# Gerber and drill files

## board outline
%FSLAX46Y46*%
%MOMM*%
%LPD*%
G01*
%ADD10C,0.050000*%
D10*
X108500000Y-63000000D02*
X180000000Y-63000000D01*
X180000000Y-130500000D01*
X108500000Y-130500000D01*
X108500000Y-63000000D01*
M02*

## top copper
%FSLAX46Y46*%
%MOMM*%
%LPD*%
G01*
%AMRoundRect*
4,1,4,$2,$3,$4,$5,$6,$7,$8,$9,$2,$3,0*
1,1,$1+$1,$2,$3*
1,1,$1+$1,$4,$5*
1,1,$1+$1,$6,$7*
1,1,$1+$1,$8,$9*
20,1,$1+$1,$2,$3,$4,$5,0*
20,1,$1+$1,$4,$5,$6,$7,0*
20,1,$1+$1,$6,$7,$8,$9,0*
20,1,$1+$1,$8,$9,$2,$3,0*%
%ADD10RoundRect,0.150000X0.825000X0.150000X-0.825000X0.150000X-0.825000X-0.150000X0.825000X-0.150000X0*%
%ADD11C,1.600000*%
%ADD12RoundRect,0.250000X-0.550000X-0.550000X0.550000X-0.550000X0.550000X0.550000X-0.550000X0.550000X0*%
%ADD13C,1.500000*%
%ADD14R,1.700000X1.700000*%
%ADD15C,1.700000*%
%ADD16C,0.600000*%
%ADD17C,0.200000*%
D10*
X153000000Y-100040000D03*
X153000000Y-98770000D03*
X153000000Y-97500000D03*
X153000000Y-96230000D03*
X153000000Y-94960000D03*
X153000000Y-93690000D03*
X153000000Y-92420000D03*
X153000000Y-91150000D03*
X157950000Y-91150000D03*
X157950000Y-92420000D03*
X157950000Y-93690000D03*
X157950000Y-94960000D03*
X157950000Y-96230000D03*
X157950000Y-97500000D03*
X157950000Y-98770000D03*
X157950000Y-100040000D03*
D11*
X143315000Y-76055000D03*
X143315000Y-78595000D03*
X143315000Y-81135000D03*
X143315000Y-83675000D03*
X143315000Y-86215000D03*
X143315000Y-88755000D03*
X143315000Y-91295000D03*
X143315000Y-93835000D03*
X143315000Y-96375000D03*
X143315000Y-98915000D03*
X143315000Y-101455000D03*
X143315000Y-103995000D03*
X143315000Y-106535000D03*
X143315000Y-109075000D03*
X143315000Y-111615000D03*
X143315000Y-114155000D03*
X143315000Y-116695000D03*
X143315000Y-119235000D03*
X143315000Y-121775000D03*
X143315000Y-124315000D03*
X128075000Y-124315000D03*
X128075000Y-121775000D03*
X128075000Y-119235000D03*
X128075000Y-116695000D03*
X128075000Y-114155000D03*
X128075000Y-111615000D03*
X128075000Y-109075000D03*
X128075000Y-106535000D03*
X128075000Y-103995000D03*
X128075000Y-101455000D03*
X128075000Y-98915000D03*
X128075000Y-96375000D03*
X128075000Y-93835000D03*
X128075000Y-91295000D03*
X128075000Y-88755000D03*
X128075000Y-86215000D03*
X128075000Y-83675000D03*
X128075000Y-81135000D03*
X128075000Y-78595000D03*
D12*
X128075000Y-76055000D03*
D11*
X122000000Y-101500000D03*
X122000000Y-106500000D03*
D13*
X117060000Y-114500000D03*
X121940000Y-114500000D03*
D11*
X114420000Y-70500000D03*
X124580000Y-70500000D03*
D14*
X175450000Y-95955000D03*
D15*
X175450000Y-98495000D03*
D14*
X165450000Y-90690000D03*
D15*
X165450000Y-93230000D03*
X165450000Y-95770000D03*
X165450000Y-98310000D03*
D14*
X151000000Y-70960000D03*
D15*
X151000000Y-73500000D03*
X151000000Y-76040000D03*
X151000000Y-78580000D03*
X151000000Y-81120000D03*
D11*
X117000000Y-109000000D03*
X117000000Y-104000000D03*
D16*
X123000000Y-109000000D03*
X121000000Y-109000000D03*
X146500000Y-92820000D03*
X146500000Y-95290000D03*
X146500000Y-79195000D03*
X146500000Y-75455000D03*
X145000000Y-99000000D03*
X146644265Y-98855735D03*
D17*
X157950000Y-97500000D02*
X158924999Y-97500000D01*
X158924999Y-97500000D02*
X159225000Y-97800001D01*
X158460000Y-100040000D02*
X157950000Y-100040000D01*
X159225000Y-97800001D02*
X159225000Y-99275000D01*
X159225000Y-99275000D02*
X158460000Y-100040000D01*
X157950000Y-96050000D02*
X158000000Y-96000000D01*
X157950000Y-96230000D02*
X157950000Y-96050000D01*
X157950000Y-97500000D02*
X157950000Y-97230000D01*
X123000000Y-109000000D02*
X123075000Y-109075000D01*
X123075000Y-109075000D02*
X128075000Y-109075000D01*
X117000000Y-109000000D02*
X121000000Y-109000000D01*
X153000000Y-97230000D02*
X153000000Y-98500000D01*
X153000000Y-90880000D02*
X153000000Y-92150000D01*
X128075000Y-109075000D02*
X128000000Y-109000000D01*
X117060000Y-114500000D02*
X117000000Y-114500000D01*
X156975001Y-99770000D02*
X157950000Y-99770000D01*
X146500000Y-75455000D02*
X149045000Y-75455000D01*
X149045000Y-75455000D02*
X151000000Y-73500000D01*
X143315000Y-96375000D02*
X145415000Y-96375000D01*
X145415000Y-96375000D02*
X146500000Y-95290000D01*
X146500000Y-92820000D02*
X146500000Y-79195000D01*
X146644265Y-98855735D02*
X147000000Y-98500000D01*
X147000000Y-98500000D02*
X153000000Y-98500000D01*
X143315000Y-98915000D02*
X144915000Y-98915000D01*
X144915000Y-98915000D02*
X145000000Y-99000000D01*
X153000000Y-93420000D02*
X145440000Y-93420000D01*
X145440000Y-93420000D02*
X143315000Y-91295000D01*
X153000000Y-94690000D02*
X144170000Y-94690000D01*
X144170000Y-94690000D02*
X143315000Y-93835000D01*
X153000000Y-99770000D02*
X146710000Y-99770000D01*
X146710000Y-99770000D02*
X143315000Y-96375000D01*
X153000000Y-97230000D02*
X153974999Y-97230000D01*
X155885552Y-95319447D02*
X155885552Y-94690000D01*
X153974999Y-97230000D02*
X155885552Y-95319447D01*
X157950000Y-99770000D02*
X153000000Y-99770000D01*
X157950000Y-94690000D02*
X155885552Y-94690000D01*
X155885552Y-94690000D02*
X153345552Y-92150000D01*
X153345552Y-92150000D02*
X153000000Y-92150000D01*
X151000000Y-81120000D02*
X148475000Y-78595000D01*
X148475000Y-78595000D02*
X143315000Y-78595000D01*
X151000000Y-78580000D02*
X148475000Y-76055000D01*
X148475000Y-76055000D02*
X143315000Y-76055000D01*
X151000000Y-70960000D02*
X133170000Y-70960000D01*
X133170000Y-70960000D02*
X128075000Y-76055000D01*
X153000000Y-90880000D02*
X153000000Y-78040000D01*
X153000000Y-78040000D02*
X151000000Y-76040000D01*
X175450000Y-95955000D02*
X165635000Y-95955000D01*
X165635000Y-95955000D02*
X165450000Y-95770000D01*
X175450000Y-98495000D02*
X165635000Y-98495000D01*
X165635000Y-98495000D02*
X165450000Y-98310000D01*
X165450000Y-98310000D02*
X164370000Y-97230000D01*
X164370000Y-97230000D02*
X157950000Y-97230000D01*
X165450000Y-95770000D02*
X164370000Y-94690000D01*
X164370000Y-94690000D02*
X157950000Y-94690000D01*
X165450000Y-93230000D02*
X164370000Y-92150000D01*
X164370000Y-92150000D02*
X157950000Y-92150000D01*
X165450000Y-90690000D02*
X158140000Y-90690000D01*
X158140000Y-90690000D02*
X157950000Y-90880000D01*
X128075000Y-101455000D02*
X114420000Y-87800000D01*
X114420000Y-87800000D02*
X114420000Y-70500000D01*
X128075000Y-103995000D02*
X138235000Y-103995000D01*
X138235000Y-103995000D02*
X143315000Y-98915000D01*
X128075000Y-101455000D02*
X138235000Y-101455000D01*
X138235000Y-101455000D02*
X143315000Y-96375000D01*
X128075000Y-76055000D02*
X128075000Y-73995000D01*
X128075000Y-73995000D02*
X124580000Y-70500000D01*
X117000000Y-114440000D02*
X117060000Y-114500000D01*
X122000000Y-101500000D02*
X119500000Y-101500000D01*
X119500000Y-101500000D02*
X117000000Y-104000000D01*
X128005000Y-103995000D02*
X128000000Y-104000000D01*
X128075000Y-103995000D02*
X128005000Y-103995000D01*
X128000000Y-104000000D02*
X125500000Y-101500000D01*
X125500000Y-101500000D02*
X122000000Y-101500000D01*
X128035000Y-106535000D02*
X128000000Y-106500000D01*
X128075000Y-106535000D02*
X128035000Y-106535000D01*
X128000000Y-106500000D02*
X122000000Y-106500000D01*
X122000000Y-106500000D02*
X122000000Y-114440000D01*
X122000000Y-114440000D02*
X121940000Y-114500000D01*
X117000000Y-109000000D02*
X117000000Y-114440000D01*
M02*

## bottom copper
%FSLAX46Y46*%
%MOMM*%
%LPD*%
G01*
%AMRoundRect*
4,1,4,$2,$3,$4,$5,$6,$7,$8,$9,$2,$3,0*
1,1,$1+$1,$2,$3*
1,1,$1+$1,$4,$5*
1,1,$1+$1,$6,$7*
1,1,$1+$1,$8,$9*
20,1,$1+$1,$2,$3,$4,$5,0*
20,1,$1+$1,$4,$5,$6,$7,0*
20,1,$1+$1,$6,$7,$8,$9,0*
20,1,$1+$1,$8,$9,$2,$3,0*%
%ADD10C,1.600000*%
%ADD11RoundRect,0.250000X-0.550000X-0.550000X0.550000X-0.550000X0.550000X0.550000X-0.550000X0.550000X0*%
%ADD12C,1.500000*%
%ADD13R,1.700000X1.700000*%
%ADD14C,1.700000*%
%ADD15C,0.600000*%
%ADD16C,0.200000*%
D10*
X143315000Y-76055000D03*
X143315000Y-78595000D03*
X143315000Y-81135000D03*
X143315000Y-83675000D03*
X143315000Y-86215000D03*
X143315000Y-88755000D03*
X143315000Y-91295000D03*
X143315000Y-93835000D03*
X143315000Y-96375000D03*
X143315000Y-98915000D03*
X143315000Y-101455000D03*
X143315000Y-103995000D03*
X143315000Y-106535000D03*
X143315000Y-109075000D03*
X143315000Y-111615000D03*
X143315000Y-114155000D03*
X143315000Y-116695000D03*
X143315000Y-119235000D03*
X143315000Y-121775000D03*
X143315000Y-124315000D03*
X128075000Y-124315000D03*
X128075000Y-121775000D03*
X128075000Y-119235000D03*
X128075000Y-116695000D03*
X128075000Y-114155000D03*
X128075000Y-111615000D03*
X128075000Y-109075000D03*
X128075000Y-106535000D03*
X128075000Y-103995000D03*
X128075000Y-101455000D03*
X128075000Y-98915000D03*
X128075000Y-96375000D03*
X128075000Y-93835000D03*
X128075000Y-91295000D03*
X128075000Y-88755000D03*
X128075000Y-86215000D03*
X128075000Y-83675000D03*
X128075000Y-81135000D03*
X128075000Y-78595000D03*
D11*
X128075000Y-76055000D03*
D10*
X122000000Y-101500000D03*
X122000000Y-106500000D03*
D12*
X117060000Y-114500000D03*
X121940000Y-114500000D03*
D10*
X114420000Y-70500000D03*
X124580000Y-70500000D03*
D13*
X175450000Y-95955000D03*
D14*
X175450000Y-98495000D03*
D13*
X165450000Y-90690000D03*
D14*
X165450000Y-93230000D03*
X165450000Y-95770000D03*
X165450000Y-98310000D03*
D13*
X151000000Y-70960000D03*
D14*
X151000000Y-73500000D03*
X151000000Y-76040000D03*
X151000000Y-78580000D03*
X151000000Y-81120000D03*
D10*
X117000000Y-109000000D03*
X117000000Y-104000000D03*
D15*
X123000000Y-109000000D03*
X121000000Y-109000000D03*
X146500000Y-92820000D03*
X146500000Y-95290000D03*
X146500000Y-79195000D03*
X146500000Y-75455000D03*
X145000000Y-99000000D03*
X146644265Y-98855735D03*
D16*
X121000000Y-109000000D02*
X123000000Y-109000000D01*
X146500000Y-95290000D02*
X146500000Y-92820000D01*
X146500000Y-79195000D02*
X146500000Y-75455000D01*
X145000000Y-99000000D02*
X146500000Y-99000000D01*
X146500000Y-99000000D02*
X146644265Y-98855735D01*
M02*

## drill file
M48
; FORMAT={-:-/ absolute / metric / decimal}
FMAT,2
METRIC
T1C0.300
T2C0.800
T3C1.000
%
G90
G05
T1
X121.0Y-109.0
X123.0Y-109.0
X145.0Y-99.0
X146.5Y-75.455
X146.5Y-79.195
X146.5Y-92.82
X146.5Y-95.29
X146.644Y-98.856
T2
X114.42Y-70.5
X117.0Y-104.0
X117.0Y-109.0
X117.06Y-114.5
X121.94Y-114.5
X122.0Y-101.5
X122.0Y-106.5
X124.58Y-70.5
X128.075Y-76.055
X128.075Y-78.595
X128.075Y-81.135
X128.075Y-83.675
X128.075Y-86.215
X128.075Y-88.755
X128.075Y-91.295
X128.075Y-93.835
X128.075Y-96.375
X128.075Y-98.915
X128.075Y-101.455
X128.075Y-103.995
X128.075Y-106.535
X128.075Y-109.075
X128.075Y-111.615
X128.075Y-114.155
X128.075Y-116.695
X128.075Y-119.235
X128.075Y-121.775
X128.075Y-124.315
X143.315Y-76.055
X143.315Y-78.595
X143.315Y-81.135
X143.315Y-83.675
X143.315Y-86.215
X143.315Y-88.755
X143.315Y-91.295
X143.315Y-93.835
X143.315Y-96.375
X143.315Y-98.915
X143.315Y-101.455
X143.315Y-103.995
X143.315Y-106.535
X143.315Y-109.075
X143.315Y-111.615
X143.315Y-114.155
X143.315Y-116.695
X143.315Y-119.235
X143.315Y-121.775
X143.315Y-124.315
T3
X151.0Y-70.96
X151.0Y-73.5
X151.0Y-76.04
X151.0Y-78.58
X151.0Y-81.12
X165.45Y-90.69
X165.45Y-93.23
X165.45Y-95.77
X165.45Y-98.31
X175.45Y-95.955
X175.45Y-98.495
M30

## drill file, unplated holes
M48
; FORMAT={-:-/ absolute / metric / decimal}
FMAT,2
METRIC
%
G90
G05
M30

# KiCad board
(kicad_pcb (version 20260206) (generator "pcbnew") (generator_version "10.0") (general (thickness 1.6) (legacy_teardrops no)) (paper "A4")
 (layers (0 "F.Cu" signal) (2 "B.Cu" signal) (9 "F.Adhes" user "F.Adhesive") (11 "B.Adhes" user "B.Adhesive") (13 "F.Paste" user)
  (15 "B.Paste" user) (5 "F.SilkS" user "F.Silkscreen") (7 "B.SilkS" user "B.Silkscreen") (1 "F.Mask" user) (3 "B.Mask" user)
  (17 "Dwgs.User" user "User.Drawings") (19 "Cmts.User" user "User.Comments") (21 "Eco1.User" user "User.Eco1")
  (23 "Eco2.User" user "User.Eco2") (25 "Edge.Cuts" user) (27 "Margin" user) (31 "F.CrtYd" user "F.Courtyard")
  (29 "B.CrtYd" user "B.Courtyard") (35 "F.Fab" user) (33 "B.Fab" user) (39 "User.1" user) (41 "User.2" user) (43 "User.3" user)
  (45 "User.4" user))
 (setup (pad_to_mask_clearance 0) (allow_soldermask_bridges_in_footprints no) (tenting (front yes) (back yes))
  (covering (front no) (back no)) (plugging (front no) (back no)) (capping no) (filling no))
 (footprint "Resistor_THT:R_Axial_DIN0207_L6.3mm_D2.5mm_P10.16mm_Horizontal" (layer "F.Cu") (at 114.42 70.5)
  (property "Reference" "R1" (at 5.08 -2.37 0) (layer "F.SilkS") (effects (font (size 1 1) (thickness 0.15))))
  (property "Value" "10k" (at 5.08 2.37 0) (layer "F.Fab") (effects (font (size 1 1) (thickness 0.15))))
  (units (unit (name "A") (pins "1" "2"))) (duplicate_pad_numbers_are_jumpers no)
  (pad "1" thru_hole circle (at 0 0) (size 1.6 1.6) (drill 0.8) (layers "*.Cu" "*.Mask") (remove_unused_layers no) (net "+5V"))
  (pad "2" thru_hole circle (at 10.16 0) (size 1.6 1.6) (drill 0.8) (layers "*.Cu" "*.Mask") (remove_unused_layers no)
   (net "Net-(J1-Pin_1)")))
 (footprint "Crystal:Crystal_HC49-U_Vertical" (layer "F.Cu") (at 117.06 114.5)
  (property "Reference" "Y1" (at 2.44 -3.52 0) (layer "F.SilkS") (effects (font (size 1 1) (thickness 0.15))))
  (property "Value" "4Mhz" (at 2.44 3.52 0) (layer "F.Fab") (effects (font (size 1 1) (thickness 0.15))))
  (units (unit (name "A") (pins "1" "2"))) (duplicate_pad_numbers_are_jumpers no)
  (pad "1" thru_hole circle (at 0 0) (size 1.5 1.5) (drill 0.8) (layers "*.Cu" "*.Mask") (remove_unused_layers no)
   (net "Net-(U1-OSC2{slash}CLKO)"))
  (pad "2" thru_hole circle (at 4.88 0) (size 1.5 1.5) (drill 0.8) (layers "*.Cu" "*.Mask") (remove_unused_layers no)
   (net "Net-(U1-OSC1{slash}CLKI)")))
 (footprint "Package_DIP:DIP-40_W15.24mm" (layer "F.Cu") (at 128.075 76.055)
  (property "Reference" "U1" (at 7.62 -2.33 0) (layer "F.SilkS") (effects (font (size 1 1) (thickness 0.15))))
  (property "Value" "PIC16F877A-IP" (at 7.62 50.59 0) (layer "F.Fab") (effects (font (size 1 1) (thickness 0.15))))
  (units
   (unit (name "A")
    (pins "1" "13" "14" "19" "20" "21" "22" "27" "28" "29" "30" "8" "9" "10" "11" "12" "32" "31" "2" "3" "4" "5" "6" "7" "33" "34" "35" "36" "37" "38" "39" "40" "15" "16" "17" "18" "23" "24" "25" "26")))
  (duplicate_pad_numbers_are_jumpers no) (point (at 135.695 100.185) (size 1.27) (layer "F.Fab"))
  (pad "1" thru_hole roundrect (at 0 0) (size 1.6 1.6) (drill 0.8) (layers "*.Cu" "*.Mask") (remove_unused_layers no)
   (roundrect_rratio 0.15625) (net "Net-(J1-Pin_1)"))
  (pad "2" thru_hole circle (at 0 2.54) (size 1.6 1.6) (drill 0.8) (layers "*.Cu" "*.Mask") (remove_unused_layers no)
   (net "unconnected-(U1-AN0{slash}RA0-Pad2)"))
  (pad "3" thru_hole circle (at 0 5.08) (size 1.6 1.6) (drill 0.8) (layers "*.Cu" "*.Mask") (remove_unused_layers no)
   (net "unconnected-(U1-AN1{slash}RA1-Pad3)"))
  (pad "4" thru_hole circle (at 0 7.62) (size 1.6 1.6) (drill 0.8) (layers "*.Cu" "*.Mask") (remove_unused_layers no)
   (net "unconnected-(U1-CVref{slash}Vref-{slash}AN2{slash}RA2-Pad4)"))
  (pad "5" thru_hole circle (at 0 10.16) (size 1.6 1.6) (drill 0.8) (layers "*.Cu" "*.Mask") (remove_unused_layers no)
   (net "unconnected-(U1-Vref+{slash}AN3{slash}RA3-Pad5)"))
  (pad "6" thru_hole circle (at 0 12.7) (size 1.6 1.6) (drill 0.8) (layers "*.Cu" "*.Mask") (remove_unused_layers no)
   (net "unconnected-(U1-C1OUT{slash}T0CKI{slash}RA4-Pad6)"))
  (pad "7" thru_hole circle (at 0 15.24) (size 1.6 1.6) (drill 0.8) (layers "*.Cu" "*.Mask") (remove_unused_layers no)
   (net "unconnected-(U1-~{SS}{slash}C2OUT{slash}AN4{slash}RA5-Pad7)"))
  (pad "8" thru_hole circle (at 0 17.78) (size 1.6 1.6) (drill 0.8) (layers "*.Cu" "*.Mask") (remove_unused_layers no)
   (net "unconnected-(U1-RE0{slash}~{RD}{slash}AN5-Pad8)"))
  (pad "9" thru_hole circle (at 0 20.32) (size 1.6 1.6) (drill 0.8) (layers "*.Cu" "*.Mask") (remove_unused_layers no)
   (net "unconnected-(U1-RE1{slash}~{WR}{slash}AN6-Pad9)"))
  (pad "10" thru_hole circle (at 0 22.86) (size 1.6 1.6) (drill 0.8) (layers "*.Cu" "*.Mask") (remove_unused_layers no)
   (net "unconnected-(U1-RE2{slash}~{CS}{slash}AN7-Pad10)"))
  (pad "11" thru_hole circle (at 0 25.4) (size 1.6 1.6) (drill 0.8) (layers "*.Cu" "*.Mask") (remove_unused_layers no) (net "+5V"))
  (pad "12" thru_hole circle (at 0 27.94) (size 1.6 1.6) (drill 0.8) (layers "*.Cu" "*.Mask") (remove_unused_layers no) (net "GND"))
  (pad "13" thru_hole circle (at 0 30.48) (size 1.6 1.6) (drill 0.8) (layers "*.Cu" "*.Mask") (remove_unused_layers no)
   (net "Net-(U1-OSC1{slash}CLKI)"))
  (pad "14" thru_hole circle (at 0 33.02) (size 1.6 1.6) (drill 0.8) (layers "*.Cu" "*.Mask") (remove_unused_layers no)
   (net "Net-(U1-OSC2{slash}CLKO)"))
  (pad "15" thru_hole circle (at 0 35.56) (size 1.6 1.6) (drill 0.8) (layers "*.Cu" "*.Mask") (remove_unused_layers no)
   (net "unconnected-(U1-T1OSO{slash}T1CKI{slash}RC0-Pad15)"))
  (pad "16" thru_hole circle (at 0 38.1) (size 1.6 1.6) (drill 0.8) (layers "*.Cu" "*.Mask") (remove_unused_layers no)
   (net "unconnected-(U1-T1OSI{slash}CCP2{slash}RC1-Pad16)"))
  (pad "17" thru_hole circle (at 0 40.64) (size 1.6 1.6) (drill 0.8) (layers "*.Cu" "*.Mask") (remove_unused_layers no)
   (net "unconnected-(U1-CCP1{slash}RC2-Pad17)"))
  (pad "18" thru_hole circle (at 0 43.18) (size 1.6 1.6) (drill 0.8) (layers "*.Cu" "*.Mask") (remove_unused_layers no)
   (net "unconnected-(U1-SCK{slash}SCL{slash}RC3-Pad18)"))
  (pad "19" thru_hole circle (at 0 45.72) (size 1.6 1.6) (drill 0.8) (layers "*.Cu" "*.Mask") (remove_unused_layers no)
   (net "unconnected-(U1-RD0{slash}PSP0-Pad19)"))
  (pad "20" thru_hole circle (at 0 48.26) (size 1.6 1.6) (drill 0.8) (layers "*.Cu" "*.Mask") (remove_unused_layers no)
   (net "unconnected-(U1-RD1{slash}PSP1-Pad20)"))
  (pad "21" thru_hole circle (at 15.24 48.26) (size 1.6 1.6) (drill 0.8) (layers "*.Cu" "*.Mask") (remove_unused_layers no)
   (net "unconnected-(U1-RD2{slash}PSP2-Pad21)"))
  (pad "22" thru_hole circle (at 15.24 45.72) (size 1.6 1.6) (drill 0.8) (layers "*.Cu" "*.Mask") (remove_unused_layers no)
   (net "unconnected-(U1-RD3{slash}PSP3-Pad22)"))
  (pad "23" thru_hole circle (at 15.24 43.18) (size 1.6 1.6) (drill 0.8) (layers "*.Cu" "*.Mask") (remove_unused_layers no)
   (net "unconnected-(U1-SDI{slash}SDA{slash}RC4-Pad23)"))
  (pad "24" thru_hole circle (at 15.24 40.64) (size 1.6 1.6) (drill 0.8) (layers "*.Cu" "*.Mask") (remove_unused_layers no)
   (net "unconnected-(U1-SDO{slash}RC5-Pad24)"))
  (pad "25" thru_hole circle (at 15.24 38.1) (size 1.6 1.6) (drill 0.8) (layers "*.Cu" "*.Mask") (remove_unused_layers no)
   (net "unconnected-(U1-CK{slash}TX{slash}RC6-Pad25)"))
  (pad "26" thru_hole circle (at 15.24 35.56) (size 1.6 1.6) (drill 0.8) (layers "*.Cu" "*.Mask") (remove_unused_layers no)
   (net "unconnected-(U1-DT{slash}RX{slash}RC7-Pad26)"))
  (pad "27" thru_hole circle (at 15.24 33.02) (size 1.6 1.6) (drill 0.8) (layers "*.Cu" "*.Mask") (remove_unused_layers no)
   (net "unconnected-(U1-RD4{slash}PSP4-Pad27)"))
  (pad "28" thru_hole circle (at 15.24 30.48) (size 1.6 1.6) (drill 0.8) (layers "*.Cu" "*.Mask") (remove_unused_layers no)
   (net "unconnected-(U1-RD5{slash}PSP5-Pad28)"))
  (pad "29" thru_hole circle (at 15.24 27.94) (size 1.6 1.6) (drill 0.8) (layers "*.Cu" "*.Mask") (remove_unused_layers no)
   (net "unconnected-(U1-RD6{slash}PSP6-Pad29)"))
  (pad "30" thru_hole circle (at 15.24 25.4) (size 1.6 1.6) (drill 0.8) (layers "*.Cu" "*.Mask") (remove_unused_layers no)
   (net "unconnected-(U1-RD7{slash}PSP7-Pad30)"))
  (pad "31" thru_hole circle (at 15.24 22.86) (size 1.6 1.6) (drill 0.8) (layers "*.Cu" "*.Mask") (remove_unused_layers no) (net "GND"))
  (pad "32" thru_hole circle (at 15.24 20.32) (size 1.6 1.6) (drill 0.8) (layers "*.Cu" "*.Mask") (remove_unused_layers no) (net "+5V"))
  (pad "33" thru_hole circle (at 15.24 17.78) (size 1.6 1.6) (drill 0.8) (layers "*.Cu" "*.Mask") (remove_unused_layers no)
   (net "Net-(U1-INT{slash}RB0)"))
  (pad "34" thru_hole circle (at 15.24 15.24) (size 1.6 1.6) (drill 0.8) (layers "*.Cu" "*.Mask") (remove_unused_layers no)
   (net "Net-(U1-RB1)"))
  (pad "35" thru_hole circle (at 15.24 12.7) (size 1.6 1.6) (drill 0.8) (layers "*.Cu" "*.Mask") (remove_unused_layers no)
   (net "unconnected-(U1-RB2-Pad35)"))
  (pad "36" thru_hole circle (at 15.24 10.16) (size 1.6 1.6) (drill 0.8) (layers "*.Cu" "*.Mask") (remove_unused_layers no)
   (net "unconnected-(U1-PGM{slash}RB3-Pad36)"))
  (pad "37" thru_hole circle (at 15.24 7.62) (size 1.6 1.6) (drill 0.8) (layers "*.Cu" "*.Mask") (remove_unused_layers no)
   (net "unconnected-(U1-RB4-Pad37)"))
  (pad "38" thru_hole circle (at 15.24 5.08) (size 1.6 1.6) (drill 0.8) (layers "*.Cu" "*.Mask") (remove_unused_layers no)
   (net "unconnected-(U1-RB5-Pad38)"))
  (pad "39" thru_hole circle (at 15.24 2.54) (size 1.6 1.6) (drill 0.8) (layers "*.Cu" "*.Mask") (remove_unused_layers no)
   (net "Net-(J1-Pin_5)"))
  (pad "40" thru_hole circle (at 15.24 0) (size 1.6 1.6) (drill 0.8) (layers "*.Cu" "*.Mask") (remove_unused_layers no)
   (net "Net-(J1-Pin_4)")))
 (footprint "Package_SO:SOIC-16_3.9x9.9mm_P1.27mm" (layer "F.Cu") (at 155.475 95.595 180)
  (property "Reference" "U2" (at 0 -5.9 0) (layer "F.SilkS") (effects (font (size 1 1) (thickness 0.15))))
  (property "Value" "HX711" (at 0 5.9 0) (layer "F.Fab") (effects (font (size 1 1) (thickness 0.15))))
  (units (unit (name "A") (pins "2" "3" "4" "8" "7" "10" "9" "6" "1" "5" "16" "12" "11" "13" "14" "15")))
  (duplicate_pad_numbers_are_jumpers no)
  (pad "1" smd roundrect (at -2.475 -4.445 180) (size 1.95 0.6) (layers "F.Cu" "F.Mask" "F.Paste") (roundrect_rratio 0.25) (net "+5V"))
  (pad "2" smd roundrect (at -2.475 -3.175 180) (size 1.95 0.6) (layers "F.Cu" "F.Mask" "F.Paste") (roundrect_rratio 0.25)
   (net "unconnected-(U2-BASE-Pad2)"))
  (pad "3" smd roundrect (at -2.475 -1.905 180) (size 1.95 0.6) (layers "F.Cu" "F.Mask" "F.Paste") (roundrect_rratio 0.25) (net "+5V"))
  (pad "4" smd roundrect (at -2.475 -0.635 180) (size 1.95 0.6) (layers "F.Cu" "F.Mask" "F.Paste") (roundrect_rratio 0.25)
   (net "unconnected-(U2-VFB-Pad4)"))
  (pad "5" smd roundrect (at -2.475 0.635 180) (size 1.95 0.6) (layers "F.Cu" "F.Mask" "F.Paste") (roundrect_rratio 0.25) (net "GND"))
  (pad "6" smd roundrect (at -2.475 1.905 180) (size 1.95 0.6) (layers "F.Cu" "F.Mask" "F.Paste") (roundrect_rratio 0.25)
   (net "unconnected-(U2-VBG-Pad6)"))
  (pad "7" smd roundrect (at -2.475 3.175 180) (size 1.95 0.6) (layers "F.Cu" "F.Mask" "F.Paste") (roundrect_rratio 0.25)
   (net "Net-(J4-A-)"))
  (pad "8" smd roundrect (at -2.475 4.445 180) (size 1.95 0.6) (layers "F.Cu" "F.Mask" "F.Paste") (roundrect_rratio 0.25)
   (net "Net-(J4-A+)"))
  (pad "9" smd roundrect (at 2.475 4.445 180) (size 1.95 0.6) (layers "F.Cu" "F.Mask" "F.Paste") (roundrect_rratio 0.25) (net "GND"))
  (pad "10" smd roundrect (at 2.475 3.175 180) (size 1.95 0.6) (layers "F.Cu" "F.Mask" "F.Paste") (roundrect_rratio 0.25) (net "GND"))
  (pad "11" smd roundrect (at 2.475 1.905 180) (size 1.95 0.6) (layers "F.Cu" "F.Mask" "F.Paste") (roundrect_rratio 0.25)
   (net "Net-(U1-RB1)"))
  (pad "12" smd roundrect (at 2.475 0.635 180) (size 1.95 0.6) (layers "F.Cu" "F.Mask" "F.Paste") (roundrect_rratio 0.25)
   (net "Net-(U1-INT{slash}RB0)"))
  (pad "13" smd roundrect (at 2.475 -0.635 180) (size 1.95 0.6) (layers "F.Cu" "F.Mask" "F.Paste") (roundrect_rratio 0.25)
   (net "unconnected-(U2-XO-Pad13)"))
  (pad "14" smd roundrect (at 2.475 -1.905 180) (size 1.95 0.6) (layers "F.Cu" "F.Mask" "F.Paste") (roundrect_rratio 0.25) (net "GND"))
  (pad "15" smd roundrect (at 2.475 -3.175 180) (size 1.95 0.6) (layers "F.Cu" "F.Mask" "F.Paste") (roundrect_rratio 0.25) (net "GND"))
  (pad "16" smd roundrect (at 2.475 -4.445 180) (size 1.95 0.6) (layers "F.Cu" "F.Mask" "F.Paste") (roundrect_rratio 0.25) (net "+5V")))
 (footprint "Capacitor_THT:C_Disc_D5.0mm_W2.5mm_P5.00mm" (layer "F.Cu") (at 117 109 90)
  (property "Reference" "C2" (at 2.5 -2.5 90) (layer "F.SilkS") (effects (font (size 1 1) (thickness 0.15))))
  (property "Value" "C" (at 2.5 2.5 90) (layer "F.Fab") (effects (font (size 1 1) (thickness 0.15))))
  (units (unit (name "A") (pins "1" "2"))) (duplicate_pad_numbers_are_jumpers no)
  (pad "1" thru_hole circle (at 0 0 90) (size 1.6 1.6) (drill 0.8) (layers "*.Cu" "*.Mask") (remove_unused_layers no)
   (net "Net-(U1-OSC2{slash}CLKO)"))
  (pad "2" thru_hole circle (at 5 0 90) (size 1.6 1.6) (drill 0.8) (layers "*.Cu" "*.Mask") (remove_unused_layers no) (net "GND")))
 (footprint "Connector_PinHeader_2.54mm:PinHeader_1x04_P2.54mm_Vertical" (layer "F.Cu") (at 165.45 90.69)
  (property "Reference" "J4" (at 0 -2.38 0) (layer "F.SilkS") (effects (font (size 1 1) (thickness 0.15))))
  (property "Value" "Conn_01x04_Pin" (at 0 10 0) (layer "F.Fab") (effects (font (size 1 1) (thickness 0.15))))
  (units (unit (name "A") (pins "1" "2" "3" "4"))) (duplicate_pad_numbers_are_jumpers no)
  (pad "1" thru_hole rect (at 0 0) (size 1.7 1.7) (drill 1) (layers "*.Cu" "*.Mask") (remove_unused_layers no) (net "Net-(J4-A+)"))
  (pad "2" thru_hole circle (at 0 2.54) (size 1.7 1.7) (drill 1) (layers "*.Cu" "*.Mask") (remove_unused_layers no) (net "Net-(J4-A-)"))
  (pad "3" thru_hole circle (at 0 5.08) (size 1.7 1.7) (drill 1) (layers "*.Cu" "*.Mask") (remove_unused_layers no) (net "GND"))
  (pad "4" thru_hole circle (at 0 7.62) (size 1.7 1.7) (drill 1) (layers "*.Cu" "*.Mask") (remove_unused_layers no) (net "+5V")))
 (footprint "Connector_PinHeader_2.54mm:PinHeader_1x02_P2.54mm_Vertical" (layer "F.Cu") (at 175.45 95.955)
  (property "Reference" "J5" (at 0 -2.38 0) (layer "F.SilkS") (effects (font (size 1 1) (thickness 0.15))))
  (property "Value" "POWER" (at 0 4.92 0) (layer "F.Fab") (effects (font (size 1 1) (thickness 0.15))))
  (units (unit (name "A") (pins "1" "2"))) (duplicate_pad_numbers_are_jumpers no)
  (pad "1" thru_hole rect (at 0 0) (size 1.7 1.7) (drill 1) (layers "*.Cu" "*.Mask") (remove_unused_layers no) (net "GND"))
  (pad "2" thru_hole circle (at 0 2.54) (size 1.7 1.7) (drill 1) (layers "*.Cu" "*.Mask") (remove_unused_layers no) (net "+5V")))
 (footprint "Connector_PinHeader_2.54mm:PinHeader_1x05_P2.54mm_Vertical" (layer "F.Cu") (at 151 70.96)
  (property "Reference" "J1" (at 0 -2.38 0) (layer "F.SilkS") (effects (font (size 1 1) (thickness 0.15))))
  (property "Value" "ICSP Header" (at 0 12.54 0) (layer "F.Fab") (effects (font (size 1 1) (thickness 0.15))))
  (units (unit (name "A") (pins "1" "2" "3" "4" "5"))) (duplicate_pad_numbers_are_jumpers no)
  (pad "1" thru_hole rect (at 0 0) (size 1.7 1.7) (drill 1) (layers "*.Cu" "*.Mask") (remove_unused_layers no) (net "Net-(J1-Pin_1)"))
  (pad "2" thru_hole circle (at 0 2.54) (size 1.7 1.7) (drill 1) (layers "*.Cu" "*.Mask") (remove_unused_layers no) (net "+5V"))
  (pad "3" thru_hole circle (at 0 5.08) (size 1.7 1.7) (drill 1) (layers "*.Cu" "*.Mask") (remove_unused_layers no) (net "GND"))
  (pad "4" thru_hole circle (at 0 7.62) (size 1.7 1.7) (drill 1) (layers "*.Cu" "*.Mask") (remove_unused_layers no) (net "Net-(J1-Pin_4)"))
  (pad "5" thru_hole circle (at 0 10.16) (size 1.7 1.7) (drill 1) (layers "*.Cu" "*.Mask") (remove_unused_layers no) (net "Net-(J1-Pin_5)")))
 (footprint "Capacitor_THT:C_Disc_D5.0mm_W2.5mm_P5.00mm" (layer "F.Cu") (at 122 106.5 90)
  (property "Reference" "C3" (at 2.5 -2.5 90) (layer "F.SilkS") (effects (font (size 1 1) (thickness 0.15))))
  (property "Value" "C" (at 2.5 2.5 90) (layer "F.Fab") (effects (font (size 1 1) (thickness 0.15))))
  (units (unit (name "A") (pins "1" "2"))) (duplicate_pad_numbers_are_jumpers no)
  (pad "1" thru_hole circle (at 0 0 90) (size 1.6 1.6) (drill 0.8) (layers "*.Cu" "*.Mask") (remove_unused_layers no)
   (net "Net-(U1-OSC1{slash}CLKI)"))
  (pad "2" thru_hole circle (at 5 0 90) (size 1.6 1.6) (drill 0.8) (layers "*.Cu" "*.Mask") (remove_unused_layers no) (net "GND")))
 (gr_rect (start 108.5 63) (end 180 130.5) (stroke (width 0.05) (type default)) (fill no) (layer "Edge.Cuts"))
 (segment (start 128.075 109.075) (end 128 109) (width 0.2) (layer "F.Cu") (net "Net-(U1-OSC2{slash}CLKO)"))
 (segment (start 123 109) (end 123.075 109.075) (width 0.2) (layer "F.Cu") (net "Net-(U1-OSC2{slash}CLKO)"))
 (segment (start 117 114.44) (end 117.06 114.5) (width 0.2) (layer "F.Cu") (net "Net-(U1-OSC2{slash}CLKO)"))
 (segment (start 117 109) (end 121 109) (width 0.2) (layer "F.Cu") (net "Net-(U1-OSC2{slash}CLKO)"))
 (segment (start 117 109) (end 117 114.44) (width 0.2) (layer "F.Cu") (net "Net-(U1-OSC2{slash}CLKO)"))
 (segment (start 117.06 114.5) (end 117 114.5) (width 0.2) (layer "F.Cu") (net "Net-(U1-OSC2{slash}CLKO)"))
 (segment (start 123.075 109.075) (end 128.075 109.075) (width 0.2) (layer "F.Cu") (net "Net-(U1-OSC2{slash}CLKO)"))
 (via (at 121 109) (size 0.6) (drill 0.3) (layers "F.Cu" "B.Cu") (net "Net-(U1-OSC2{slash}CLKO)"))
 (via (at 123 109) (size 0.6) (drill 0.3) (layers "F.Cu" "B.Cu") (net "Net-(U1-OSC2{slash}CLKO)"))
 (segment (start 121 109) (end 123 109) (width 0.2) (layer "B.Cu") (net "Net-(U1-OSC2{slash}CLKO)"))
 (segment (start 165.635 95.955) (end 165.45 95.77) (width 0.2) (layer "F.Cu") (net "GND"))
 (segment (start 146.644265 98.855735) (end 147 98.5) (width 0.2) (layer "F.Cu") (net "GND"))
 (segment (start 143.315 98.915) (end 144.915 98.915) (width 0.2) (layer "F.Cu") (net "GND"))
 (segment (start 128 104) (end 125.5 101.5) (width 0.2) (layer "F.Cu") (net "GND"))
 (segment (start 155.885552 94.69) (end 153.345552 92.15) (width 0.2) (layer "F.Cu") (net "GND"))
 (segment (start 153 90.88) (end 153 78.04) (width 0.2) (layer "F.Cu") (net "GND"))
 (segment (start 165.45 95.77) (end 164.37 94.69) (width 0.2) (layer "F.Cu") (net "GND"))
 (segment (start 153.345552 92.15) (end 153 92.15) (width 0.2) (layer "F.Cu") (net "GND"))
 (segment (start 128.075 103.995) (end 138.235 103.995) (width 0.2) (layer "F.Cu") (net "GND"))
 (segment (start 138.235 103.995) (end 143.315 98.915) (width 0.2) (layer "F.Cu") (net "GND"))
 (segment (start 147 98.5) (end 153 98.5) (width 0.2) (layer "F.Cu") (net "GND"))
 (segment (start 153 78.04) (end 151 76.04) (width 0.2) (layer "F.Cu") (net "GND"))
 (segment (start 125.5 101.5) (end 122 101.5) (width 0.2) (layer "F.Cu") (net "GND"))
 (segment (start 175.45 95.955) (end 165.635 95.955) (width 0.2) (layer "F.Cu") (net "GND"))
 (segment (start 164.37 94.69) (end 157.95 94.69) (width 0.2) (layer "F.Cu") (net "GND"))
 (segment (start 128.075 103.995) (end 128.005 103.995) (width 0.2) (layer "F.Cu") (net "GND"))
 (segment (start 119.5 101.5) (end 117 104) (width 0.2) (layer "F.Cu") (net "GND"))
 (segment (start 128.005 103.995) (end 128 104) (width 0.2) (layer "F.Cu") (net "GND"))
 (segment (start 153 97.23) (end 153.974999 97.23) (width 0.2) (layer "F.Cu") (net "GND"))
 (segment (start 155.885552 95.319447) (end 155.885552 94.69) (width 0.2) (layer "F.Cu") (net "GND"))
 (segment (start 122 101.5) (end 119.5 101.5) (width 0.2) (layer "F.Cu") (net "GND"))
 (segment (start 153.974999 97.23) (end 155.885552 95.319447) (width 0.2) (layer "F.Cu") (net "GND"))
 (segment (start 153 90.88) (end 153 92.15) (width 0.2) (layer "F.Cu") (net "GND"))
 (segment (start 144.915 98.915) (end 145 99) (width 0.2) (layer "F.Cu") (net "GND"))
 (segment (start 153 97.23) (end 153 98.5) (width 0.2) (layer "F.Cu") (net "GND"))
 (segment (start 157.95 94.69) (end 155.885552 94.69) (width 0.2) (layer "F.Cu") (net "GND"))
 (via (at 146.644265 98.855735) (size 0.6) (drill 0.3) (layers "F.Cu" "B.Cu") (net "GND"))
 (via (at 145 99) (size 0.6) (drill 0.3) (layers "F.Cu" "B.Cu") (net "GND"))
 (segment (start 145 99) (end 146.5 99) (width 0.2) (layer "B.Cu") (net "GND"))
 (segment (start 146.5 99) (end 146.644265 98.855735) (width 0.2) (layer "B.Cu") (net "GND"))
 (segment (start 128 106.5) (end 122 106.5) (width 0.2) (layer "F.Cu") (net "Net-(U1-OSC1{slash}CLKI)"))
 (segment (start 122 106.5) (end 122 114.44) (width 0.2) (layer "F.Cu") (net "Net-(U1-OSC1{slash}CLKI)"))
 (segment (start 122 114.44) (end 121.94 114.5) (width 0.2) (layer "F.Cu") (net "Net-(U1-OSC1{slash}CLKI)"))
 (segment (start 128.075 106.535) (end 128.035 106.535) (width 0.2) (layer "F.Cu") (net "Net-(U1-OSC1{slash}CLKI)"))
 (segment (start 128.035 106.535) (end 128 106.5) (width 0.2) (layer "F.Cu") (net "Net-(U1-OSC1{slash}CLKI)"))
 (segment (start 148.475 76.055) (end 143.315 76.055) (width 0.2) (layer "F.Cu") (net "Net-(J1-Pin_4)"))
 (segment (start 151 78.58) (end 148.475 76.055) (width 0.2) (layer "F.Cu") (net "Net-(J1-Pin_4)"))
 (segment (start 128.075 73.995) (end 124.58 70.5) (width 0.2) (layer "F.Cu") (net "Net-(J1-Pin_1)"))
 (segment (start 128.075 76.055) (end 128.075 73.995) (width 0.2) (layer "F.Cu") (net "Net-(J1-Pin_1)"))
 (segment (start 133.17 70.96) (end 128.075 76.055) (width 0.2) (layer "F.Cu") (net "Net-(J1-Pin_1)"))
 (segment (start 151 70.96) (end 133.17 70.96) (width 0.2) (layer "F.Cu") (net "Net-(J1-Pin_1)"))
 (segment (start 128.075 101.455) (end 114.42 87.8) (width 0.2) (layer "F.Cu") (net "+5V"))
 (segment (start 159.225 99.275) (end 158.46 100.04) (width 0.2) (layer "F.Cu") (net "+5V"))
 (segment (start 146.71 99.77) (end 143.315 96.375) (width 0.2) (layer "F.Cu") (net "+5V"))
 (segment (start 157.95 97.5) (end 158.924999 97.5) (width 0.2) (layer "F.Cu") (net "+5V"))
 (segment (start 159.225 97.800001) (end 159.225 99.275) (width 0.2) (layer "F.Cu") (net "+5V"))
 (segment (start 146.5 75.455) (end 149.045 75.455) (width 0.2) (layer "F.Cu") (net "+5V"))
 (segment (start 165.635 98.495) (end 165.45 98.31) (width 0.2) (layer "F.Cu") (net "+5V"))
 (segment (start 149.045 75.455) (end 151 73.5) (width 0.2) (layer "F.Cu") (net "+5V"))
 (segment (start 158.46 100.04) (end 157.95 100.04) (width 0.2) (layer "F.Cu") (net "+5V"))
 (segment (start 156.975001 99.77) (end 157.95 99.77) (width 0.2) (layer "F.Cu") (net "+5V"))
 (segment (start 175.45 98.495) (end 165.635 98.495) (width 0.2) (layer "F.Cu") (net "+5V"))
 (segment (start 165.45 98.31) (end 164.37 97.23) (width 0.2) (layer "F.Cu") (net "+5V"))
 (segment (start 138.235 101.455) (end 143.315 96.375) (width 0.2) (layer "F.Cu") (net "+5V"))
 (segment (start 158.924999 97.5) (end 159.225 97.800001) (width 0.2) (layer "F.Cu") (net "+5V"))
 (segment (start 128.075 101.455) (end 138.235 101.455) (width 0.2) (layer "F.Cu") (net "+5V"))
 (segment (start 146.5 92.82) (end 146.5 79.195) (width 0.2) (layer "F.Cu") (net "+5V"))
 (segment (start 145.415 96.375) (end 146.5 95.29) (width 0.2) (layer "F.Cu") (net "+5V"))
 (segment (start 153 99.77) (end 146.71 99.77) (width 0.2) (layer "F.Cu") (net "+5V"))
 (segment (start 157.95 97.5) (end 157.95 97.23) (width 0.2) (layer "F.Cu") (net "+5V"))
 (segment (start 114.42 87.8) (end 114.42 70.5) (width 0.2) (layer "F.Cu") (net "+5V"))
 (segment (start 143.315 96.375) (end 145.415 96.375) (width 0.2) (layer "F.Cu") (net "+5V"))
 (segment (start 157.95 99.77) (end 153 99.77) (width 0.2) (layer "F.Cu") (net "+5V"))
 (segment (start 164.37 97.23) (end 157.95 97.23) (width 0.2) (layer "F.Cu") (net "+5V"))
 (via (at 146.5 75.455) (size 0.6) (drill 0.3) (layers "F.Cu" "B.Cu") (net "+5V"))
 (via (at 146.5 92.82) (size 0.6) (drill 0.3) (layers "F.Cu" "B.Cu") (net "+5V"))
 (via (at 146.5 95.29) (size 0.6) (drill 0.3) (layers "F.Cu" "B.Cu") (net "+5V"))
 (via (at 146.5 79.195) (size 0.6) (drill 0.3) (layers "F.Cu" "B.Cu") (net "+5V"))
 (segment (start 146.5 79.195) (end 146.5 75.455) (width 0.2) (layer "B.Cu") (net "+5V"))
 (segment (start 146.5 95.29) (end 146.5 92.82) (width 0.2) (layer "B.Cu") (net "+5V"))
 (segment (start 148.475 78.595) (end 143.315 78.595) (width 0.2) (layer "F.Cu") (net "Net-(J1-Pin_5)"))
 (segment (start 151 81.12) (end 148.475 78.595) (width 0.2) (layer "F.Cu") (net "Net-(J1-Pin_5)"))
 (segment (start 165.45 90.69) (end 158.14 90.69) (width 0.2) (layer "F.Cu") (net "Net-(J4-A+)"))
 (segment (start 158.14 90.69) (end 157.95 90.88) (width 0.2) (layer "F.Cu") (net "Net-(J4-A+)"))
 (segment (start 165.45 93.23) (end 164.37 92.15) (width 0.2) (layer "F.Cu") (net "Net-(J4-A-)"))
 (segment (start 164.37 92.15) (end 157.95 92.15) (width 0.2) (layer "F.Cu") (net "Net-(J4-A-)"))
 (segment (start 145.44 93.42) (end 143.315 91.295) (width 0.2) (layer "F.Cu") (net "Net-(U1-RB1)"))
 (segment (start 153 93.42) (end 145.44 93.42) (width 0.2) (layer "F.Cu") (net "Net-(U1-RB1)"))
 (segment (start 153 94.69) (end 144.17 94.69) (width 0.2) (layer "F.Cu") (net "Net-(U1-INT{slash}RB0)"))
 (segment (start 144.17 94.69) (end 143.315 93.835) (width 0.2) (layer "F.Cu") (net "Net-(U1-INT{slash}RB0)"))
 (segment (start 157.95 96.23) (end 157.95 96.05) (width 0.2) (layer "F.Cu") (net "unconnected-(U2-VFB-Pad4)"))
 (segment (start 157.95 96.05) (end 158 96) (width 0.2) (layer "F.Cu") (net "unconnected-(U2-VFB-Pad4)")))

